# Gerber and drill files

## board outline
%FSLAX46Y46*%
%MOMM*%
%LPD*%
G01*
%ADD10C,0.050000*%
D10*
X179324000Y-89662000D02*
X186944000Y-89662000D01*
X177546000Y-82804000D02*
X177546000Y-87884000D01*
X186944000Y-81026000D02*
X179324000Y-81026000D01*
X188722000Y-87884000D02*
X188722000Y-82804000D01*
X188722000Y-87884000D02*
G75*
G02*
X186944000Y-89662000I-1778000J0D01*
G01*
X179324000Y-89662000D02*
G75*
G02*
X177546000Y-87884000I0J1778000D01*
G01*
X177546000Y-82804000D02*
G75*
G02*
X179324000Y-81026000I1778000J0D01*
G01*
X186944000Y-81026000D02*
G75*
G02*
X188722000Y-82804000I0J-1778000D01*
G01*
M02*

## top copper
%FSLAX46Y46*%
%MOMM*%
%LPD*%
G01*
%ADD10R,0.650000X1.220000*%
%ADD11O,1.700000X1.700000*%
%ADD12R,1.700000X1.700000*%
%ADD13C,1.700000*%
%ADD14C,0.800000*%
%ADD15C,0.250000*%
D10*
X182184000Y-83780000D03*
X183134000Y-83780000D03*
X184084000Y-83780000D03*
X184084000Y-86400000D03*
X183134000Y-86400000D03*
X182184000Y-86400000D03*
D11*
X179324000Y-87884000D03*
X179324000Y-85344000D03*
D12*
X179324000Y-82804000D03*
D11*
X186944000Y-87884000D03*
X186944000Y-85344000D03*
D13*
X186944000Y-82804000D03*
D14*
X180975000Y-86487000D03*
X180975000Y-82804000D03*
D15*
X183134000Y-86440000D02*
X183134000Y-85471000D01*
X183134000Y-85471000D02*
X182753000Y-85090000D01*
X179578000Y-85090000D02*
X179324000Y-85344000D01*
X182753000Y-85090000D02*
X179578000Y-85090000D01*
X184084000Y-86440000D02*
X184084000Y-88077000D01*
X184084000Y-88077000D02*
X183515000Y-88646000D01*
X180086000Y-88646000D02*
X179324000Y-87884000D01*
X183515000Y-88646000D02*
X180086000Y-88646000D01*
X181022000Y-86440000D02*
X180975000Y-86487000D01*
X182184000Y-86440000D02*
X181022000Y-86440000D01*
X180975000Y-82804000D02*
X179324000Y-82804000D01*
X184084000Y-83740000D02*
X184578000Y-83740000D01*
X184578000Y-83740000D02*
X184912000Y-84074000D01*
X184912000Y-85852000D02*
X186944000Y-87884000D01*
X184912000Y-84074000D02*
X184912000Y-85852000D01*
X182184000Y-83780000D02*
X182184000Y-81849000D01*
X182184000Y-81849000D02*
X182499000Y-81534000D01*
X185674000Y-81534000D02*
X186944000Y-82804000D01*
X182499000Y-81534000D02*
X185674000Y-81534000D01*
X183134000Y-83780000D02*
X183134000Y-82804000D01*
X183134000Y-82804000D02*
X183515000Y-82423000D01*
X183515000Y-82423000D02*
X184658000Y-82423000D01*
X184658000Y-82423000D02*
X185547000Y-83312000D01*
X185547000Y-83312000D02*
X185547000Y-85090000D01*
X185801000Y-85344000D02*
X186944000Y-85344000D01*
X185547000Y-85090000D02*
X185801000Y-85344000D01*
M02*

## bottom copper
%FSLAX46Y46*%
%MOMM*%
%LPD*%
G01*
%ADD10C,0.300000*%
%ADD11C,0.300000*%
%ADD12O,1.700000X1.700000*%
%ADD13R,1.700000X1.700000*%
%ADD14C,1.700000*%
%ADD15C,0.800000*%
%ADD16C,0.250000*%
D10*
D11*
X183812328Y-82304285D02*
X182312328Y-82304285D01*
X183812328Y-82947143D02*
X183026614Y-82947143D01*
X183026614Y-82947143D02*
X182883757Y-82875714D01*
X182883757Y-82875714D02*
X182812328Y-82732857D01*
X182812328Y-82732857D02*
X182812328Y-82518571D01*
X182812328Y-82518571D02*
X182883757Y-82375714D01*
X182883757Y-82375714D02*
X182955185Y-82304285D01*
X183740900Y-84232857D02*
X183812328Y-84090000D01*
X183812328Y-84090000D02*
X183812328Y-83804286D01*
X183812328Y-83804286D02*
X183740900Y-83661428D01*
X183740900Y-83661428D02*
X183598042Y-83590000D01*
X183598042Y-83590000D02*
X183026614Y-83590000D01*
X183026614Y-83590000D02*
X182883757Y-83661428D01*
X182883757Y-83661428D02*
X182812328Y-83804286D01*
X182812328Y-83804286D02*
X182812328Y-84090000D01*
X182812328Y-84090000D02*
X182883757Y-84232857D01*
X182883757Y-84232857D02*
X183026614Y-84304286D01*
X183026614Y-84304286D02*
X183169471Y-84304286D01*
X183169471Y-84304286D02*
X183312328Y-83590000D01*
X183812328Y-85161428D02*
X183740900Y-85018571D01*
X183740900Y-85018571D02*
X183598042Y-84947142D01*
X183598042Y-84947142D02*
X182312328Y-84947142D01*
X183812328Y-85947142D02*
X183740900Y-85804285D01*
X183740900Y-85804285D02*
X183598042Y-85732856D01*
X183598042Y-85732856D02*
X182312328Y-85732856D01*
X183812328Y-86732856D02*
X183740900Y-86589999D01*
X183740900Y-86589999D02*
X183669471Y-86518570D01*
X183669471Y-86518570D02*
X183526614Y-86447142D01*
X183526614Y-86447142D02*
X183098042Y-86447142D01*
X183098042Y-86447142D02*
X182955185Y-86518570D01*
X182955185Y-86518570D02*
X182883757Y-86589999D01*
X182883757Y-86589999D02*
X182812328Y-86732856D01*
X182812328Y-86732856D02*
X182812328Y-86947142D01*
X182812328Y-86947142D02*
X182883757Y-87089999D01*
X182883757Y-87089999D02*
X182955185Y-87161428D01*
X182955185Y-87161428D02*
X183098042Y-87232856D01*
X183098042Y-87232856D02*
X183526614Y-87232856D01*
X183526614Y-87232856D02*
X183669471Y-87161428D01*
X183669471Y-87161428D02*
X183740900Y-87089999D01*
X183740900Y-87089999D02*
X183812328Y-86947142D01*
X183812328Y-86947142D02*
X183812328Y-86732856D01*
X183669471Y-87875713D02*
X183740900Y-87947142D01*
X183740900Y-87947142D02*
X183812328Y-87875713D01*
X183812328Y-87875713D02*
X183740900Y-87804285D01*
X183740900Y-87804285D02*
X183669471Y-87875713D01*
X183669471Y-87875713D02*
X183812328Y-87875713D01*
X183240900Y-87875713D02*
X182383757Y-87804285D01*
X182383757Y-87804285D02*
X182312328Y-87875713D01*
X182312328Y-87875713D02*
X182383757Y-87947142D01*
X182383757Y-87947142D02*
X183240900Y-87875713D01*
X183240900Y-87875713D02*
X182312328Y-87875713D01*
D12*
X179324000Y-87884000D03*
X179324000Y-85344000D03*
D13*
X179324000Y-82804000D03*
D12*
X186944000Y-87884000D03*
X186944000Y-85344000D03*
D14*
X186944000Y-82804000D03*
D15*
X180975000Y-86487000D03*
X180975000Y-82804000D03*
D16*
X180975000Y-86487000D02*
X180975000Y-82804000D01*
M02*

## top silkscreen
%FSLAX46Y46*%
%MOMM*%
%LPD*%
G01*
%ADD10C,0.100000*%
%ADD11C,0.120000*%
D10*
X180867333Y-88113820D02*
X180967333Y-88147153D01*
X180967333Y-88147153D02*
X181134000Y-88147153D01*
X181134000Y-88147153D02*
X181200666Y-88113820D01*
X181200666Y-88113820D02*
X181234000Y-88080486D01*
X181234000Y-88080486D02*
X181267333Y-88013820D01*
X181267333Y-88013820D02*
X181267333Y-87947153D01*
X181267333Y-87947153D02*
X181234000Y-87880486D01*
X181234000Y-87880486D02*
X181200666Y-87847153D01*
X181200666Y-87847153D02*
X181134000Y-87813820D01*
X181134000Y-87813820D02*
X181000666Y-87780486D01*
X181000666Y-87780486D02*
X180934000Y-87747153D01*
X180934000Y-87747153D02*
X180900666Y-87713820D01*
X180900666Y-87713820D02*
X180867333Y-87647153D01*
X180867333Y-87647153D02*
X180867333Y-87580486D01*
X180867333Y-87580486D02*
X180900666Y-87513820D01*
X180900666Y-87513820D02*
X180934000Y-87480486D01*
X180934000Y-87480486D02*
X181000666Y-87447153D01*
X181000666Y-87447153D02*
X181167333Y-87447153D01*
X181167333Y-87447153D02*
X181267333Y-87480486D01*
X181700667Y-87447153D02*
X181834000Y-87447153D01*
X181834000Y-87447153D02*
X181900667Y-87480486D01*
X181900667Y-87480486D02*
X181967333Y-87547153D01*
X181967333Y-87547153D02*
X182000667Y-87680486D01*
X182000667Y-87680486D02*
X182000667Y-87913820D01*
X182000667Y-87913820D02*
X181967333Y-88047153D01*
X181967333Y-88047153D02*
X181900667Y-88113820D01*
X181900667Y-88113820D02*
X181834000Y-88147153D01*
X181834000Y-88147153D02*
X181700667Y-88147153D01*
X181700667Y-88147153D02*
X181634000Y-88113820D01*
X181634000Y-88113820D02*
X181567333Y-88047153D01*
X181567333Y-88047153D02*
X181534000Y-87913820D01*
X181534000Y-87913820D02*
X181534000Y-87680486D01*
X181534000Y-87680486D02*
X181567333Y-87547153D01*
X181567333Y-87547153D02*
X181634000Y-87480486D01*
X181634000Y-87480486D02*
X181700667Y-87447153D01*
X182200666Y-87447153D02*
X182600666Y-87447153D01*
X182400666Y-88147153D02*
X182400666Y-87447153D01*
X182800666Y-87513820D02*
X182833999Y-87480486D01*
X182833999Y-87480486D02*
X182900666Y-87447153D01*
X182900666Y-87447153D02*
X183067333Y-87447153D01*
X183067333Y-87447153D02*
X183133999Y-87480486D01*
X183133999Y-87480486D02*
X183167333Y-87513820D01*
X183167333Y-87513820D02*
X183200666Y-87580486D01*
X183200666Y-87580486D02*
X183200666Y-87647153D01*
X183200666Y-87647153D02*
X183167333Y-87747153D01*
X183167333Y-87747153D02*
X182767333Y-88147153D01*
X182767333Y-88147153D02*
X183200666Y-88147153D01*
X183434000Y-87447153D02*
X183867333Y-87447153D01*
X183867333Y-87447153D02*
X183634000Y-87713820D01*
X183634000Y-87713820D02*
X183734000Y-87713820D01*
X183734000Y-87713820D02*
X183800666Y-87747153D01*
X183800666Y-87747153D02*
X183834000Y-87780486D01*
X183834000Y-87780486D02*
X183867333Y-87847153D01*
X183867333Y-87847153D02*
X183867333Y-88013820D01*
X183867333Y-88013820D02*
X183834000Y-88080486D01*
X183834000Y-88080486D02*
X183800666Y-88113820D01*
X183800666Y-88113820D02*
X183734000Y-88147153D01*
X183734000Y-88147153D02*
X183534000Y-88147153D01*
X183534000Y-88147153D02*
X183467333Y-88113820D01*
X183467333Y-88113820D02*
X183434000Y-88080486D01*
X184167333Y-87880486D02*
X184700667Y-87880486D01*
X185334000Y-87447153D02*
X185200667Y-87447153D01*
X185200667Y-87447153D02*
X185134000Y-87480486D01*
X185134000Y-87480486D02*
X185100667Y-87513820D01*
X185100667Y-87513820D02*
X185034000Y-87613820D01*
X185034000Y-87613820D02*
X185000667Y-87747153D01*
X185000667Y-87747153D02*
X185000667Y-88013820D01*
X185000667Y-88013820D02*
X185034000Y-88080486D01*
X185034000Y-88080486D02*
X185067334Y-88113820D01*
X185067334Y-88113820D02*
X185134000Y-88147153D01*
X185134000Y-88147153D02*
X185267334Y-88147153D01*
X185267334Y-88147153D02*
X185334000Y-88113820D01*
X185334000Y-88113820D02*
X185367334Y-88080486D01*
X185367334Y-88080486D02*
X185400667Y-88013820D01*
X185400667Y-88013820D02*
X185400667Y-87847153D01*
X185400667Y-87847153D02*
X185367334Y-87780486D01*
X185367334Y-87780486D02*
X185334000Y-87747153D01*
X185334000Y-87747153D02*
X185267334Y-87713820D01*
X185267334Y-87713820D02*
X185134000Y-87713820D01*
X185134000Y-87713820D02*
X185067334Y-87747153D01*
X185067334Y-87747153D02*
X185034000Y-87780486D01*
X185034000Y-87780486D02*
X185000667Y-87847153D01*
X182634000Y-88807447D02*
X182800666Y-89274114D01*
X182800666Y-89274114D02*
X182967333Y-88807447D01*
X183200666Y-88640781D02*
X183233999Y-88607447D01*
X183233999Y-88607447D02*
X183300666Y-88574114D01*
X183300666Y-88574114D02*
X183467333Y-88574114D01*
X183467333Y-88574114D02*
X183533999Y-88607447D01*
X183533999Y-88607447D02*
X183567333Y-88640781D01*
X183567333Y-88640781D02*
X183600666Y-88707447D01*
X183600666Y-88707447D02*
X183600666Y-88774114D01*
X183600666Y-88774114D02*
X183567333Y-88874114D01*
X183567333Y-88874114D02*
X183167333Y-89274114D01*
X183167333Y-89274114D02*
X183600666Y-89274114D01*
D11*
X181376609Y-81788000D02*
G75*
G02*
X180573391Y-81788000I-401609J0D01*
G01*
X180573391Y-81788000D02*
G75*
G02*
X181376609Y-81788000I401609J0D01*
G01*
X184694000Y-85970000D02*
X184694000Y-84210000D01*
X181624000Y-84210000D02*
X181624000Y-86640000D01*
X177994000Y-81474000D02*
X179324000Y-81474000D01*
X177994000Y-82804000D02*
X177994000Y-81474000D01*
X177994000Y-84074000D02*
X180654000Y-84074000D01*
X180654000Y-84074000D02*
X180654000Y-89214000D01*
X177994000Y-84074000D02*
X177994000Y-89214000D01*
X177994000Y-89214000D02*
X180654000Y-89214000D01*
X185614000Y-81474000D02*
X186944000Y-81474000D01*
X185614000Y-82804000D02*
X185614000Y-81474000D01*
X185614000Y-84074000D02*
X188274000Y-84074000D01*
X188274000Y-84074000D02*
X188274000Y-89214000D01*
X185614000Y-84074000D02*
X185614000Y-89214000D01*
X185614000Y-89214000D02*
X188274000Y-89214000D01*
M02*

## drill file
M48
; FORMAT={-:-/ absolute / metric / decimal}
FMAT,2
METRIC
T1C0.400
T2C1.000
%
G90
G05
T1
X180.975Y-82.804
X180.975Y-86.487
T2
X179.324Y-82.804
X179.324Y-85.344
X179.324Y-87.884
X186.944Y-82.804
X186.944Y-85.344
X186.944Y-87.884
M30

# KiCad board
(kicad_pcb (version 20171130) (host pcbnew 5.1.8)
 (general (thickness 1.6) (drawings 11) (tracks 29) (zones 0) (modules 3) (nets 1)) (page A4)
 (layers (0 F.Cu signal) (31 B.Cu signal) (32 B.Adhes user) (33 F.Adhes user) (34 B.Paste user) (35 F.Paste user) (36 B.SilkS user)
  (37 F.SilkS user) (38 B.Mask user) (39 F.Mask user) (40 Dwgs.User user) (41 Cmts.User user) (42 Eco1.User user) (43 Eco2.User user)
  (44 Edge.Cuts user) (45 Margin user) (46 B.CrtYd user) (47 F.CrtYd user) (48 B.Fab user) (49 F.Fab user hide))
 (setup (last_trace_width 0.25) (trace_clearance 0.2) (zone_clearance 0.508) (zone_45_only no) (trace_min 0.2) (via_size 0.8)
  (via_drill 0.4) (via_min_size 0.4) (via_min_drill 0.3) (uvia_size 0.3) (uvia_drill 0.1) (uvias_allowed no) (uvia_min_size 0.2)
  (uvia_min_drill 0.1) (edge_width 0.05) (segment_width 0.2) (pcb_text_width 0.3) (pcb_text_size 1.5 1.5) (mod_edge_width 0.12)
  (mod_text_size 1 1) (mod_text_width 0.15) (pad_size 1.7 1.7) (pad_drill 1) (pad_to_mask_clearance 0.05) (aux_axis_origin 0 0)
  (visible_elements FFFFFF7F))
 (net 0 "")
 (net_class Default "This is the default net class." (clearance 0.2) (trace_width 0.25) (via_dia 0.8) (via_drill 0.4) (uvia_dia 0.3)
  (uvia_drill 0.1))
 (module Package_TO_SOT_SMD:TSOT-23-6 (layer F.Cu) (at 183.134 85.09 90)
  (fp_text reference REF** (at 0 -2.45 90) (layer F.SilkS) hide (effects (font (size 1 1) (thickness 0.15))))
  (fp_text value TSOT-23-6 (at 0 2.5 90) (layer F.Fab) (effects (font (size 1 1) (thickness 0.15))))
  (fp_line (start -0.88 1.56) (end 0.88 1.56) (layer F.SilkS) (width 0.12))
  (fp_line (start 0.88 -1.51) (end -1.55 -1.51) (layer F.SilkS) (width 0.12))
  (pad 6 smd rect (at 1.31 -0.95 90) (size 1.22 0.65) (layers F.Cu F.Paste F.Mask))
  (pad 5 smd rect (at 1.31 0 90) (size 1.22 0.65) (layers F.Cu F.Paste F.Mask))
  (pad 4 smd rect (at 1.31 0.95 90) (size 1.22 0.65) (layers F.Cu F.Paste F.Mask))
  (pad 3 smd rect (at -1.31 0.95 90) (size 1.22 0.65) (layers F.Cu F.Paste F.Mask))
  (pad 2 smd rect (at -1.31 0 90) (size 1.22 0.65) (layers F.Cu F.Paste F.Mask))
  (pad 1 smd rect (at -1.31 -0.95 90) (size 1.22 0.65) (layers F.Cu F.Paste F.Mask)))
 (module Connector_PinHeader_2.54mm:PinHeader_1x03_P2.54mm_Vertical (layer F.Cu) (at 179.324 82.804)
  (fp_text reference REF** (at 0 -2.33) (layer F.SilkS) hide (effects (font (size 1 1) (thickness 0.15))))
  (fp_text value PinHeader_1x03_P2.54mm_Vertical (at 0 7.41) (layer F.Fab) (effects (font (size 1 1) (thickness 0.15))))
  (fp_line (start -1.33 -1.33) (end 0 -1.33) (layer F.SilkS) (width 0.12))
  (fp_line (start -1.33 0) (end -1.33 -1.33) (layer F.SilkS) (width 0.12))
  (fp_line (start -1.33 1.27) (end 1.33 1.27) (layer F.SilkS) (width 0.12))
  (fp_line (start 1.33 1.27) (end 1.33 6.41) (layer F.SilkS) (width 0.12))
  (fp_line (start -1.33 1.27) (end -1.33 6.41) (layer F.SilkS) (width 0.12))
  (fp_line (start -1.33 6.41) (end 1.33 6.41) (layer F.SilkS) (width 0.12))
  (pad 3 thru_hole oval (at 0 5.08) (size 1.7 1.7) (drill 1) (layers *.Cu *.Mask))
  (pad 2 thru_hole oval (at 0 2.54) (size 1.7 1.7) (drill 1) (layers *.Cu *.Mask))
  (pad 1 thru_hole rect (at 0 0) (size 1.7 1.7) (drill 1) (layers *.Cu *.Mask)))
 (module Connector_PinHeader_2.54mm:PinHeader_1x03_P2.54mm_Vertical (layer F.Cu) (at 186.944 82.804)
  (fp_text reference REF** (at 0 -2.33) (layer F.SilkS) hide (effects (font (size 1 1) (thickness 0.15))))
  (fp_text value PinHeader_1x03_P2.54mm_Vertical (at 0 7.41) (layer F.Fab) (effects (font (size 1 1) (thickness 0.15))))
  (fp_line (start -1.33 -1.33) (end 0 -1.33) (layer F.SilkS) (width 0.12))
  (fp_line (start -1.33 0) (end -1.33 -1.33) (layer F.SilkS) (width 0.12))
  (fp_line (start -1.33 1.27) (end 1.33 1.27) (layer F.SilkS) (width 0.12))
  (fp_line (start 1.33 1.27) (end 1.33 6.41) (layer F.SilkS) (width 0.12))
  (fp_line (start -1.33 1.27) (end -1.33 6.41) (layer F.SilkS) (width 0.12))
  (fp_line (start -1.33 6.41) (end 1.33 6.41) (layer F.SilkS) (width 0.12))
  (pad 4 thru_hole oval (at 0 5.08) (size 1.7 1.7) (drill 1) (layers *.Cu *.Mask))
  (pad 5 thru_hole oval (at 0 2.54) (size 1.7 1.7) (drill 1) (layers *.Cu *.Mask))
  (pad 6 thru_hole circle (at 0 0) (size 1.7 1.7) (drill 1) (layers *.Cu *.Mask)))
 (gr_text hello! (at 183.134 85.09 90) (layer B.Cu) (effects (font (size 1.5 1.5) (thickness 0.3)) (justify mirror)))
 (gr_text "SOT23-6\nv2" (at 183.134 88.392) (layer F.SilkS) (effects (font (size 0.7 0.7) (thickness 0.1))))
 (gr_line (start 179.324 89.662) (end 186.944 89.662) (layer Edge.Cuts) (width 0.05))
 (gr_line (start 177.546 82.804) (end 177.546 87.884) (layer Edge.Cuts) (width 0.05))
 (gr_line (start 186.944 81.026) (end 179.324 81.026) (layer Edge.Cuts) (width 0.05))
 (gr_line (start 188.722 87.884) (end 188.722 82.804) (layer Edge.Cuts) (width 0.05))
 (gr_arc (start 186.944 87.884) (end 186.944 89.662) (angle -90) (layer Edge.Cuts) (width 0.05))
 (gr_arc (start 179.324 87.884) (end 177.546 87.884) (angle -90) (layer Edge.Cuts) (width 0.05))
 (gr_arc (start 179.324 82.804) (end 179.324 81.026) (angle -90) (layer Edge.Cuts) (width 0.05))
 (gr_arc (start 186.944 82.804) (end 188.722 82.804) (angle -90) (layer Edge.Cuts) (width 0.05))
 (gr_circle (center 180.975 81.788) (end 181.356 81.661) (layer F.SilkS) (width 0.12))
 (segment (start 183.134 86.44) (end 183.134 85.471) (width 0.25) (layer F.Cu) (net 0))
 (segment (start 183.134 85.471) (end 182.753 85.09) (width 0.25) (layer F.Cu) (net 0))
 (segment (start 179.578 85.09) (end 179.324 85.344) (width 0.25) (layer F.Cu) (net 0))
 (segment (start 182.753 85.09) (end 179.578 85.09) (width 0.25) (layer F.Cu) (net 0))
 (segment (start 184.084 86.44) (end 184.084 88.077) (width 0.25) (layer F.Cu) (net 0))
 (segment (start 184.084 88.077) (end 183.515 88.646) (width 0.25) (layer F.Cu) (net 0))
 (segment (start 180.086 88.646) (end 179.324 87.884) (width 0.25) (layer F.Cu) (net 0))
 (segment (start 183.515 88.646) (end 180.086 88.646) (width 0.25) (layer F.Cu) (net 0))
 (via (at 180.975 86.487) (size 0.8) (drill 0.4) (layers F.Cu B.Cu) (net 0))
 (via (at 180.975 82.804) (size 0.8) (drill 0.4) (layers F.Cu B.Cu) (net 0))
 (segment (start 181.022 86.44) (end 180.975 86.487) (width 0.25) (layer F.Cu) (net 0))
 (segment (start 182.184 86.44) (end 181.022 86.44) (width 0.25) (layer F.Cu) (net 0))
 (segment (start 180.975 82.804) (end 179.324 82.804) (width 0.25) (layer F.Cu) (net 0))
 (segment (start 180.975 86.487) (end 180.975 82.804) (width 0.25) (layer B.Cu) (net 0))
 (segment (start 184.084 83.74) (end 184.578 83.74) (width 0.25) (layer F.Cu) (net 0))
 (segment (start 184.578 83.74) (end 184.912 84.074) (width 0.25) (layer F.Cu) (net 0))
 (segment (start 184.912 85.852) (end 186.944 87.884) (width 0.25) (layer F.Cu) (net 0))
 (segment (start 184.912 84.074) (end 184.912 85.852) (width 0.25) (layer F.Cu) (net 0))
 (segment (start 182.184 83.78) (end 182.184 81.849) (width 0.25) (layer F.Cu) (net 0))
 (segment (start 182.184 81.849) (end 182.499 81.534) (width 0.25) (layer F.Cu) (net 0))
 (segment (start 185.674 81.534) (end 186.944 82.804) (width 0.25) (layer F.Cu) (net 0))
 (segment (start 182.499 81.534) (end 185.674 81.534) (width 0.25) (layer F.Cu) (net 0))
 (segment (start 183.134 83.78) (end 183.134 82.804) (width 0.25) (layer F.Cu) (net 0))
 (segment (start 183.134 82.804) (end 183.515 82.423) (width 0.25) (layer F.Cu) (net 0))
 (segment (start 183.515 82.423) (end 184.658 82.423) (width 0.25) (layer F.Cu) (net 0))
 (segment (start 184.658 82.423) (end 185.547 83.312) (width 0.25) (layer F.Cu) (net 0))
 (segment (start 185.547 83.312) (end 185.547 85.09) (width 0.25) (layer F.Cu) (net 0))
 (segment (start 185.801 85.344) (end 186.944 85.344) (width 0.25) (layer F.Cu) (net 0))
 (segment (start 185.547 85.09) (end 185.801 85.344) (width 0.25) (layer F.Cu) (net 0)))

